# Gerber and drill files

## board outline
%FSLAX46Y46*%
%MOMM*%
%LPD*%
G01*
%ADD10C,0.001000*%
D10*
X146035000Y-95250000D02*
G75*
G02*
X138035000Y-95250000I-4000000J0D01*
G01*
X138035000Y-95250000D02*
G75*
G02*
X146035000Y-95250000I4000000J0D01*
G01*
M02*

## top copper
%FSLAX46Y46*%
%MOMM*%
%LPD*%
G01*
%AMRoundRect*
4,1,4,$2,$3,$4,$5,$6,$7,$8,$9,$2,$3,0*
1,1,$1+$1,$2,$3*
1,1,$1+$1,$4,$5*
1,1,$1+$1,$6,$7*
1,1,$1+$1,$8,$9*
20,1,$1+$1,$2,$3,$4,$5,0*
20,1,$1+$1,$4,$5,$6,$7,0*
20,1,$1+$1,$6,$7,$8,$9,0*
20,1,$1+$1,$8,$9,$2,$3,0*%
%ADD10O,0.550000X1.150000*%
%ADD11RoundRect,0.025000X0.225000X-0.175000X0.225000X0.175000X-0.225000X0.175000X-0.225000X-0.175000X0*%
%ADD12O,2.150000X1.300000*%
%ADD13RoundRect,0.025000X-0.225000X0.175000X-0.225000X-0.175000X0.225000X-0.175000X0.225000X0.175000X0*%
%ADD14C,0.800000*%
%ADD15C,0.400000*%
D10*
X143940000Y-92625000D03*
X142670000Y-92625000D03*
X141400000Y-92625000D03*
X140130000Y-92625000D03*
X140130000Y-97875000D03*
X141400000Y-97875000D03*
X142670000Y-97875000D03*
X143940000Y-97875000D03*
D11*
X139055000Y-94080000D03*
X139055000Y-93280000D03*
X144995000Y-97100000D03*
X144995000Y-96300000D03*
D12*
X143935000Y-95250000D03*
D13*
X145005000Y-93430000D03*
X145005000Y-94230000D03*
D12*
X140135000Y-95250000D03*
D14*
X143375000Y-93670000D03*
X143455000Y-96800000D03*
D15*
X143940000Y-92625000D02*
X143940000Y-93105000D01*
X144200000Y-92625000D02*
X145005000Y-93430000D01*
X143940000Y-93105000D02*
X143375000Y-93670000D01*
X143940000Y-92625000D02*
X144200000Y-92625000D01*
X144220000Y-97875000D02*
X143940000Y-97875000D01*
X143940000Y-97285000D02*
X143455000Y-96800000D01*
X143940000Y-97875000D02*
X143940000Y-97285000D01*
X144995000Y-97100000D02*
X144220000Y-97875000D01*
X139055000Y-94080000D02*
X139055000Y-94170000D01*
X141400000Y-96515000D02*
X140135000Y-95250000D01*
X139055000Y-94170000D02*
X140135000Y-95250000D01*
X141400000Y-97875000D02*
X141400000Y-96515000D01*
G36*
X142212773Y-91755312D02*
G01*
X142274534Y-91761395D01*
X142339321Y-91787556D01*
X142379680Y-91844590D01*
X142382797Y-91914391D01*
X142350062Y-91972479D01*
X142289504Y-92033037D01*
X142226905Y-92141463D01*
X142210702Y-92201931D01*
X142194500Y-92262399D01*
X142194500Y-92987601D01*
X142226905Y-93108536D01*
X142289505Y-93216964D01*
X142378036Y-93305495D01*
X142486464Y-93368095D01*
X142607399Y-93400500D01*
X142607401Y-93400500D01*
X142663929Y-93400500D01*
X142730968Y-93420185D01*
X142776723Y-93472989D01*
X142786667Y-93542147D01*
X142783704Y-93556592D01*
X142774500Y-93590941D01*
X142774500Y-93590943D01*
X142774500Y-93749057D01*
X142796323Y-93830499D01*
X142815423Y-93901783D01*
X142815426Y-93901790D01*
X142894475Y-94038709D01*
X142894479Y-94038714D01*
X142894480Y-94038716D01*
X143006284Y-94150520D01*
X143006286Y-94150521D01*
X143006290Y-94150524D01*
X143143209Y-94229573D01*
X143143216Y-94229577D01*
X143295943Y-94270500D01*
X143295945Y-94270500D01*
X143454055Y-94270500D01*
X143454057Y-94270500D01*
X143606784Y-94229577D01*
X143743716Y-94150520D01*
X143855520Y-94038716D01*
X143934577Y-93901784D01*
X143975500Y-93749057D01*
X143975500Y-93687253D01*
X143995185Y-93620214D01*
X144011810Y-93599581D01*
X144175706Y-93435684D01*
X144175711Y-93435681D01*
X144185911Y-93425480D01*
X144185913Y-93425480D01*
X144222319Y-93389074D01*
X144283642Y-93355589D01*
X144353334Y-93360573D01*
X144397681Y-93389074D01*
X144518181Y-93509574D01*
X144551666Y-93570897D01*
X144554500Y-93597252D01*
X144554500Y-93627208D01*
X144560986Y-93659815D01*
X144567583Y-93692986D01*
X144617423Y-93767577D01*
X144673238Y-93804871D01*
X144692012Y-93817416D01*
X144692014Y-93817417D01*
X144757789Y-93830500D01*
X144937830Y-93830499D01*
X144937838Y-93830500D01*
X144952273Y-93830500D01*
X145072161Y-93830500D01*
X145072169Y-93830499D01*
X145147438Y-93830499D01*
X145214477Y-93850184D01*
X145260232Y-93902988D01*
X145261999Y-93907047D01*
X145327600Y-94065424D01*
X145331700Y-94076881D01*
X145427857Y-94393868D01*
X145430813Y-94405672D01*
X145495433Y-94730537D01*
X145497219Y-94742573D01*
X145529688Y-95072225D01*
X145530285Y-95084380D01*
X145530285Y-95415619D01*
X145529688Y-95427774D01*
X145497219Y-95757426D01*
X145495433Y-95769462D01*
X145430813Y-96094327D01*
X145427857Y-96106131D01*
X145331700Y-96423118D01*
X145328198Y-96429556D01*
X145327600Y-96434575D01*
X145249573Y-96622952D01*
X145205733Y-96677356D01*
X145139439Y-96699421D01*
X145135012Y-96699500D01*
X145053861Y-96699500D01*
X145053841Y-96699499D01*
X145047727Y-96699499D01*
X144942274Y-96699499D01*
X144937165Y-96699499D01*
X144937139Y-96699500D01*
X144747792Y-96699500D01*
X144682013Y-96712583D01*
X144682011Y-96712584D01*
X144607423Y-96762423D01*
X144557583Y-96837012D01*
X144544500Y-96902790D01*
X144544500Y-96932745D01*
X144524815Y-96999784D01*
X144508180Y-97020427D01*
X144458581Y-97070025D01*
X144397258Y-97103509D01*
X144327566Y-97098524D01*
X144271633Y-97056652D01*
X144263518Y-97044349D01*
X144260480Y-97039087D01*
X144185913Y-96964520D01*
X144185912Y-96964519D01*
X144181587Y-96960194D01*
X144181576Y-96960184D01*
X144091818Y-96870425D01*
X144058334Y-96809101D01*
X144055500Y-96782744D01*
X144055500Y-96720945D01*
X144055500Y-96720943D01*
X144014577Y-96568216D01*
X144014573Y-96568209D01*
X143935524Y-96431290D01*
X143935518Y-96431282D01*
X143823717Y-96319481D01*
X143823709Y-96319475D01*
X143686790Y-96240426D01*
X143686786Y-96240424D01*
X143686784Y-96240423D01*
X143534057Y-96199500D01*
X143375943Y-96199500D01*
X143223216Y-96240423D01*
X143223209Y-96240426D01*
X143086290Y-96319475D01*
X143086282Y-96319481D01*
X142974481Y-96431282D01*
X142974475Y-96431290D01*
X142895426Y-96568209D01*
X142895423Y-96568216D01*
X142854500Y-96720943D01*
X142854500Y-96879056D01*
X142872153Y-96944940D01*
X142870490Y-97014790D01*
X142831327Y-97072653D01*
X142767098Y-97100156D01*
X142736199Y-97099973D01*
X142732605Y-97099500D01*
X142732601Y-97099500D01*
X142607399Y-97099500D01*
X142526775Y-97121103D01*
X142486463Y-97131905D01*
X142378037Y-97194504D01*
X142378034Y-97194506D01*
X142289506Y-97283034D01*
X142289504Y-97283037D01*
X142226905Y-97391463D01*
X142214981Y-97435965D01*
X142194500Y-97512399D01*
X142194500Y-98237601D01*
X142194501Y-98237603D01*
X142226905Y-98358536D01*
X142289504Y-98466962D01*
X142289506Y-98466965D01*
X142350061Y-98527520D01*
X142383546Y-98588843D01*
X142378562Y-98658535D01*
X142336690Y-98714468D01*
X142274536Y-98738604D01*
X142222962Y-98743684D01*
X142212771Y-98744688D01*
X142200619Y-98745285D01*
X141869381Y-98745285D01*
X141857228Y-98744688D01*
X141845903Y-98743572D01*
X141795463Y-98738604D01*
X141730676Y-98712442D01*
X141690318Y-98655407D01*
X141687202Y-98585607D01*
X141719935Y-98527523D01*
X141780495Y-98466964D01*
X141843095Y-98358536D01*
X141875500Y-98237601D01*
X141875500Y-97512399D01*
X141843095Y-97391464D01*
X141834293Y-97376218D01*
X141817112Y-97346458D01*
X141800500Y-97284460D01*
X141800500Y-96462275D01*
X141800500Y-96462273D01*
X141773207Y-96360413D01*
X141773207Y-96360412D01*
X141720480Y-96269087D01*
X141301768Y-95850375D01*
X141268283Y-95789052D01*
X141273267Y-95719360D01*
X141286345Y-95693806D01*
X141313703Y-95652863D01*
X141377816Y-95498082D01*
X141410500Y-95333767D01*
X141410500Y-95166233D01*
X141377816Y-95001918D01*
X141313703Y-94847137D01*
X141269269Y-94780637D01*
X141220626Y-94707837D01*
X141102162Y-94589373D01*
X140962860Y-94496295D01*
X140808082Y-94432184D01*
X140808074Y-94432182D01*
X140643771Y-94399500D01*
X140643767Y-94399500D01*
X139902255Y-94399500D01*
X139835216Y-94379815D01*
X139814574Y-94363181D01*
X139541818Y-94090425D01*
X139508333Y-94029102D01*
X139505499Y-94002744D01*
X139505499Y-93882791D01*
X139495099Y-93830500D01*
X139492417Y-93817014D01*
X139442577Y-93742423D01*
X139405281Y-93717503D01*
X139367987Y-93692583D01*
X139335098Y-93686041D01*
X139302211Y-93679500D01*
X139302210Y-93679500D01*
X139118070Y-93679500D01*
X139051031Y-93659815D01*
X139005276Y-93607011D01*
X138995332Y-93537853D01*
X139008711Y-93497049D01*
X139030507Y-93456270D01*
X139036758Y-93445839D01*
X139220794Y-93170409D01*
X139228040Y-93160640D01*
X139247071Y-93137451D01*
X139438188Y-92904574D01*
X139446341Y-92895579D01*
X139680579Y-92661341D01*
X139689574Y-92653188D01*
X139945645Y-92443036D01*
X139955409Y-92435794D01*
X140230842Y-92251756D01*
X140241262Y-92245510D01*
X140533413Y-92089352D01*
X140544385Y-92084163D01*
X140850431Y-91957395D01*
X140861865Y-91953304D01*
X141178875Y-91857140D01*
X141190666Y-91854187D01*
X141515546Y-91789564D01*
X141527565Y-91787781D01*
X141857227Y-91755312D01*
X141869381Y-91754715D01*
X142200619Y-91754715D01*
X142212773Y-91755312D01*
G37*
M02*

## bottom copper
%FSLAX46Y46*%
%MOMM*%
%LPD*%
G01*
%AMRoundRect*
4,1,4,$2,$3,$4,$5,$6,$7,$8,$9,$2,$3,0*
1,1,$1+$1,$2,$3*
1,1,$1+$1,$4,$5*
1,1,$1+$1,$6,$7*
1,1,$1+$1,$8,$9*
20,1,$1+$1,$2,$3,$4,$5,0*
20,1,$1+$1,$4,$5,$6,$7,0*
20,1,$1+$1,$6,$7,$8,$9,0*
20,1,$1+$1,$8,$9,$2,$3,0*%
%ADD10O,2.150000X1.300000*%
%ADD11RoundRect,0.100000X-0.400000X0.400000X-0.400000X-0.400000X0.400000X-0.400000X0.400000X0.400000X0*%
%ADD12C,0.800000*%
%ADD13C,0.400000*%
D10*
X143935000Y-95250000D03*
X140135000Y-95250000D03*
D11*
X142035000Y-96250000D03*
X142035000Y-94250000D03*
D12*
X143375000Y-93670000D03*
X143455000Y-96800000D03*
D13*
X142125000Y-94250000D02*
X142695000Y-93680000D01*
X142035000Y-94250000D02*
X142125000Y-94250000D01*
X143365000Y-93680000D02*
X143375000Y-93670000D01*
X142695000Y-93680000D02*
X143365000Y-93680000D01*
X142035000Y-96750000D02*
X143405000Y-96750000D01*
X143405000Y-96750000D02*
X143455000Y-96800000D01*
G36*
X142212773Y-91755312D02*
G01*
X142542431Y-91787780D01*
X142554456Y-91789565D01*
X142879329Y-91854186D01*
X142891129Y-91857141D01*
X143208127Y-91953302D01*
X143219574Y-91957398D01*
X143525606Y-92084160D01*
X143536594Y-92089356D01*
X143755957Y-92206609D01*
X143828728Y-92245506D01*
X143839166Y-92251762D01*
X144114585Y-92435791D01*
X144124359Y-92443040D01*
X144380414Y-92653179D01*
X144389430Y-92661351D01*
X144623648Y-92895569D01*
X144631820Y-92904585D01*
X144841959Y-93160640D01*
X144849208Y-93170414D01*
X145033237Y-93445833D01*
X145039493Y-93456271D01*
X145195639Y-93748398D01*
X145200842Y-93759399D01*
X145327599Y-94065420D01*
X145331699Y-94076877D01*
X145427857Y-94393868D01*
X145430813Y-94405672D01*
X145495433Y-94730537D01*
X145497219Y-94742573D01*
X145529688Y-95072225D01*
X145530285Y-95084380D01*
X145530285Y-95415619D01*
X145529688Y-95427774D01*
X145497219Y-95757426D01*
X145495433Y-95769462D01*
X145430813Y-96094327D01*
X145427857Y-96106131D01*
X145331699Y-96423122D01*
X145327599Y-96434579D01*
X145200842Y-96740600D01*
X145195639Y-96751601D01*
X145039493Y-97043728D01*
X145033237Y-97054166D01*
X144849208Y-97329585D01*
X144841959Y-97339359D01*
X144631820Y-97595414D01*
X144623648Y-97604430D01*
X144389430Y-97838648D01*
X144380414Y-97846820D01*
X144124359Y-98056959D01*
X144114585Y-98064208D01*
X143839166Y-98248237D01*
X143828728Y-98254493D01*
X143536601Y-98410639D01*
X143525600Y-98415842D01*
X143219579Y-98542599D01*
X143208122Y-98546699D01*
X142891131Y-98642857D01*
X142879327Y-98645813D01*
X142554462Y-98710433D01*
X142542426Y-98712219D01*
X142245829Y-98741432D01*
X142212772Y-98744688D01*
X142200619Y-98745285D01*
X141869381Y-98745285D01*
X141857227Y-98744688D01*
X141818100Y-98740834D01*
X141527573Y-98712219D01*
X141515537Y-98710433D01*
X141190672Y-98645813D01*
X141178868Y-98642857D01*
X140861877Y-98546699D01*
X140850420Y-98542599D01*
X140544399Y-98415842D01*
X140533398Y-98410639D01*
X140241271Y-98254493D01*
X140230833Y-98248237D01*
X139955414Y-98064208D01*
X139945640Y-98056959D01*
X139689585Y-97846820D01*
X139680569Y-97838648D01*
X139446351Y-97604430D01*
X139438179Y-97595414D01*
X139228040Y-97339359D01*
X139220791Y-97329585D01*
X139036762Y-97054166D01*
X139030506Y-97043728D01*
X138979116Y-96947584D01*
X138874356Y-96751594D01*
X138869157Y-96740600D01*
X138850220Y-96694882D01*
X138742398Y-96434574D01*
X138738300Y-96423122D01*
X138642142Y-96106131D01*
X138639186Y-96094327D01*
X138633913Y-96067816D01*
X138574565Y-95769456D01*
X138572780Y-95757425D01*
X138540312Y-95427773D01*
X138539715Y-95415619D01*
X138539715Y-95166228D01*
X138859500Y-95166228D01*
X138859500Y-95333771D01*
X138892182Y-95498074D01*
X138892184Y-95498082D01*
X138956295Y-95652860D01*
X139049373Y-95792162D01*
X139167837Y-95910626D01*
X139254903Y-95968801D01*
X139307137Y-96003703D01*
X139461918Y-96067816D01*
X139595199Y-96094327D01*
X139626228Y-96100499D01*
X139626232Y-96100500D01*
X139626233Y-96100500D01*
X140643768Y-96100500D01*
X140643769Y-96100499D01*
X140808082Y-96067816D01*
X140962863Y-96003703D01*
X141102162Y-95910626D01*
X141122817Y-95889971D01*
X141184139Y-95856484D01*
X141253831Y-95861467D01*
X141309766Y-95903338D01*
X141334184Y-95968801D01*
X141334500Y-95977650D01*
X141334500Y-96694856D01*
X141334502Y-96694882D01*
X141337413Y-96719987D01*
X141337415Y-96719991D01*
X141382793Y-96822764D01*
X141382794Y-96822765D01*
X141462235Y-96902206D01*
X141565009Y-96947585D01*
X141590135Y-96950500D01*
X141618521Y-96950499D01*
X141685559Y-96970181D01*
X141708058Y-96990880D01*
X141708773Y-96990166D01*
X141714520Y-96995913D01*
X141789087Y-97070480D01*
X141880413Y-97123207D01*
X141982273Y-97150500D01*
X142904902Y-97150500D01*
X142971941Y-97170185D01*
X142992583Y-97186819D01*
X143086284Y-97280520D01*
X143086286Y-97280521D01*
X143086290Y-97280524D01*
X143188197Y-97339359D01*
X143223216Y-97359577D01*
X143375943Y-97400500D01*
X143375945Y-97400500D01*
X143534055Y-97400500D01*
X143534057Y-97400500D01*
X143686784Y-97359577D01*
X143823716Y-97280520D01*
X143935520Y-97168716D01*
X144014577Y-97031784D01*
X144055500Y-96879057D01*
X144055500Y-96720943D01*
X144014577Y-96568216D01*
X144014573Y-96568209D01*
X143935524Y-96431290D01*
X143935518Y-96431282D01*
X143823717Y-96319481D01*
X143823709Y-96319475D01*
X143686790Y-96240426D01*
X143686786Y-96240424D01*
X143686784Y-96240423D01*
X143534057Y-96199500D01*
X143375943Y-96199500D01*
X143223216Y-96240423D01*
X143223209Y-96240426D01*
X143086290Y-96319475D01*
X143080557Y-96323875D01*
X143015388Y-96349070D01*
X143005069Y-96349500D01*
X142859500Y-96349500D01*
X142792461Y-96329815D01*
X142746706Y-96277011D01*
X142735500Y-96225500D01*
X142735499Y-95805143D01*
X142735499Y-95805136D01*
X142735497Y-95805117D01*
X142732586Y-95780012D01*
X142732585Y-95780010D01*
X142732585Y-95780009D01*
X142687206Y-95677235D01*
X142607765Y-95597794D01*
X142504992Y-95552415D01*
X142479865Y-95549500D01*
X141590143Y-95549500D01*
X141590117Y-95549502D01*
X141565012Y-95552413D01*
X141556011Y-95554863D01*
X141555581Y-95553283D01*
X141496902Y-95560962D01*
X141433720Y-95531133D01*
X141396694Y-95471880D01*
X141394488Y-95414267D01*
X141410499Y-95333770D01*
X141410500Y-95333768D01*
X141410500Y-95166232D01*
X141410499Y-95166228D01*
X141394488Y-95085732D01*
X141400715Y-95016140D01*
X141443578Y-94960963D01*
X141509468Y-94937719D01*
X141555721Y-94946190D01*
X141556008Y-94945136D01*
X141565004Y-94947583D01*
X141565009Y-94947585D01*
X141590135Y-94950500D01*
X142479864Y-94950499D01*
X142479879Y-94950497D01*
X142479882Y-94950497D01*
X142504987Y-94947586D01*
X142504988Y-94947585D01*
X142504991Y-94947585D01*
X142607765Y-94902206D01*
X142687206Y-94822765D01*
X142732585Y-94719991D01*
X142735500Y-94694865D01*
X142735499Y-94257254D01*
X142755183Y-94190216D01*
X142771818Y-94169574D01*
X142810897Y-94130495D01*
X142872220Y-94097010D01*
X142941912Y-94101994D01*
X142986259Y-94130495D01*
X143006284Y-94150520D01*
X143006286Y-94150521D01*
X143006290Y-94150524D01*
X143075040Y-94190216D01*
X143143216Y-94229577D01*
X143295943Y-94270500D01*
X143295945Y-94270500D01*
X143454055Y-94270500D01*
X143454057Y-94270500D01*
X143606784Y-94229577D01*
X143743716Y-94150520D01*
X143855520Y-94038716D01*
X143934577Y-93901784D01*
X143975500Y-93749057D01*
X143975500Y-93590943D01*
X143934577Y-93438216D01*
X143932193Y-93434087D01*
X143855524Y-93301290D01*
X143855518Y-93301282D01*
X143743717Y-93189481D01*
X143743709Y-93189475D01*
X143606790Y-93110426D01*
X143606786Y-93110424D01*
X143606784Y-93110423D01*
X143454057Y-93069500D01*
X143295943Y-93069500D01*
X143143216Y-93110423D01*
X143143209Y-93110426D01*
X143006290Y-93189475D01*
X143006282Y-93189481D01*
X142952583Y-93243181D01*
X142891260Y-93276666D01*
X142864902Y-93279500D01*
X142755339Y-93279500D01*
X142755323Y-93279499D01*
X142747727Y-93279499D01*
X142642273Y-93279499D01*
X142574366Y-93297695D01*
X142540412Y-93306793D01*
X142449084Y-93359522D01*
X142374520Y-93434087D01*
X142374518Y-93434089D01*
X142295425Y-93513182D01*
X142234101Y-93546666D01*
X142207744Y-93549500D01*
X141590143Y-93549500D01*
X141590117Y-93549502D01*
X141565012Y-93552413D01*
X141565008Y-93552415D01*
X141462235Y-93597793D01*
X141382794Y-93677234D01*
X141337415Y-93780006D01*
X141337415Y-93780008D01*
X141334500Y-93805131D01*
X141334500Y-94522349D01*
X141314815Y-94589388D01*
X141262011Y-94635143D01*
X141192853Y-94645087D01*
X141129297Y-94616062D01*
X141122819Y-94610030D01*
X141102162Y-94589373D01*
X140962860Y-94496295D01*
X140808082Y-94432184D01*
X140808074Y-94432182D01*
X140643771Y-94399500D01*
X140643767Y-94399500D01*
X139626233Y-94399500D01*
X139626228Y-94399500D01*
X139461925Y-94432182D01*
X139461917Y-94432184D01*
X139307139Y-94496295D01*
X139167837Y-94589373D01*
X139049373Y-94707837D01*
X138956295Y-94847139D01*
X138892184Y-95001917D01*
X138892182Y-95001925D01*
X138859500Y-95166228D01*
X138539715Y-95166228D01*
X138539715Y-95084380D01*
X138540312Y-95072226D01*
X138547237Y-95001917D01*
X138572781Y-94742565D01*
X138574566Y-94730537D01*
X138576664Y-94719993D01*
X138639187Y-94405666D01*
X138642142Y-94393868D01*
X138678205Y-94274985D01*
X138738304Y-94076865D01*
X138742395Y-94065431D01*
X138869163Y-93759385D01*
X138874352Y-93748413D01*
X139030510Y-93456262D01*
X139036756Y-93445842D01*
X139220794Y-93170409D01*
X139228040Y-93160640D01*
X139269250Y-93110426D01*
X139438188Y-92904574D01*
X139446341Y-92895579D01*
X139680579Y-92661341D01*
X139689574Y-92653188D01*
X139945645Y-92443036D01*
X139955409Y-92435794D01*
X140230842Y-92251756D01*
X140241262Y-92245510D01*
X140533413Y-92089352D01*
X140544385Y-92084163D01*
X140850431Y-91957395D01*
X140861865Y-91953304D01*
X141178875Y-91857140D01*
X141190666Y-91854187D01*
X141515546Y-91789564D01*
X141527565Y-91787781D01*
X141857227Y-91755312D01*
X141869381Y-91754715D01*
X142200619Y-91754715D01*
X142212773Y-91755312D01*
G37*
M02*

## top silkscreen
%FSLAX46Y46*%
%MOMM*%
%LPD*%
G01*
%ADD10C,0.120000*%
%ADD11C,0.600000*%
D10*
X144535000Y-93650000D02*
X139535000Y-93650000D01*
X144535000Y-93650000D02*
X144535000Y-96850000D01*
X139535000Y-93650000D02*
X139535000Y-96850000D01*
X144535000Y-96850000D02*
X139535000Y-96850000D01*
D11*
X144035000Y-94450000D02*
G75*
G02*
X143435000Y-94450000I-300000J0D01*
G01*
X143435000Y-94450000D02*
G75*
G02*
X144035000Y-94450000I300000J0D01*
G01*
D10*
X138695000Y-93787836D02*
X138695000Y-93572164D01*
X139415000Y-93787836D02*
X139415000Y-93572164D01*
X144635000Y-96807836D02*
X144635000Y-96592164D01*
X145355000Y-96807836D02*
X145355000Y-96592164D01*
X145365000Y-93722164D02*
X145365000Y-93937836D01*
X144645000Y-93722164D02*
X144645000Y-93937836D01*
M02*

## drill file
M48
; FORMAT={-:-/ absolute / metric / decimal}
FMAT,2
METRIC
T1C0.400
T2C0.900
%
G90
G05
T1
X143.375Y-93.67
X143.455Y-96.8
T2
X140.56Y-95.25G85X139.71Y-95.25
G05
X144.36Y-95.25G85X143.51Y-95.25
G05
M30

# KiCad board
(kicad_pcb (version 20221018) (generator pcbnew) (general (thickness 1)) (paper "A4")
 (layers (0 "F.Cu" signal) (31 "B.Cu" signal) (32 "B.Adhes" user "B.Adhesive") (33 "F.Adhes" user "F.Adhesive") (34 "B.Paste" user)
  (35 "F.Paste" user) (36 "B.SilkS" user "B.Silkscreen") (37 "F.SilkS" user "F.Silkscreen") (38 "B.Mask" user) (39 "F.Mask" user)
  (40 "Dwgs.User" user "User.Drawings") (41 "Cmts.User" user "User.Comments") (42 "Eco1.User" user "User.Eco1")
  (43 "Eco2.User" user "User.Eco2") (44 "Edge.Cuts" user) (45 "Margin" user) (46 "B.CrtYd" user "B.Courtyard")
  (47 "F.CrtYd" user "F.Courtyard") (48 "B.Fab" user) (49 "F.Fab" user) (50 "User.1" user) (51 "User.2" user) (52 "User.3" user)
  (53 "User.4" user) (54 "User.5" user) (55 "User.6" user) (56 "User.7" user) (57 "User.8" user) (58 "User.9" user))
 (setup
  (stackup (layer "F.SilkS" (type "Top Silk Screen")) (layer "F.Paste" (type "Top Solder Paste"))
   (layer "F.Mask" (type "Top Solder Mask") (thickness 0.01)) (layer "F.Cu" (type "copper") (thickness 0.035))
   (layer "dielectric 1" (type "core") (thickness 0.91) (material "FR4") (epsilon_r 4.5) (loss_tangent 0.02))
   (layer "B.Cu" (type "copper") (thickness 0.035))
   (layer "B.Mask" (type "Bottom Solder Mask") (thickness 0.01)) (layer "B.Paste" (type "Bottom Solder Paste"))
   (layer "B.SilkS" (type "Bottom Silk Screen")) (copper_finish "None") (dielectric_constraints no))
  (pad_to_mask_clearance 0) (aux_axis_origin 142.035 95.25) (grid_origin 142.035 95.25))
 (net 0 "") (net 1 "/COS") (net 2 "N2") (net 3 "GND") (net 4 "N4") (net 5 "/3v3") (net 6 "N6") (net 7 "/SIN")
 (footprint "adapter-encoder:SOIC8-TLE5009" (layer "F.Cu") (at 142.035 95.25 -90)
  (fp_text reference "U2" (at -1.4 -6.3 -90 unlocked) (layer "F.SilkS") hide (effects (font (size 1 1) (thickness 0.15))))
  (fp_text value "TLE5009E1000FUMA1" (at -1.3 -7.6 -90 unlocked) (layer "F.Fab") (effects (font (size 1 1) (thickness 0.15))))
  (fp_line (start -1.6 -2.5) (end -1.6 2.5) (stroke (width 0.12) (type default)) (layer "F.SilkS"))
  (fp_line (start -1.6 -2.5) (end 1.6 -2.5) (stroke (width 0.12) (type default)) (layer "F.SilkS"))
  (fp_line (start -1.6 2.5) (end 1.6 2.5) (stroke (width 0.12) (type default)) (layer "F.SilkS"))
  (fp_line (start 1.6 -2.5) (end 1.6 2.5) (stroke (width 0.12) (type default)) (layer "F.SilkS"))
  (fp_circle (center -0.8 -1.7) (end -0.5 -1.7) (stroke (width 0.6) (type default)) (fill none) (layer "F.SilkS"))
  (pad "1" smd oval (at -2.625 -1.905) (size 0.55 1.15) (layers "F.Cu" "F.Paste" "F.Mask") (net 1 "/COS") (solder_mask_margin 0.0508))
  (pad "2" smd oval (at -2.625 -0.635) (size 0.55 1.15) (layers "F.Cu" "F.Paste" "F.Mask") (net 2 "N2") (solder_mask_margin 0.0508))
  (pad "3" smd oval (at -2.625 0.635) (size 0.55 1.15) (layers "F.Cu" "F.Paste" "F.Mask") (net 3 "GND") (solder_mask_margin 0.0508))
  (pad "4" smd oval (at -2.625 1.905) (size 0.55 1.15) (layers "F.Cu" "F.Paste" "F.Mask") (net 3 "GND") (solder_mask_margin 0.0508))
  (pad "5" smd oval (at 2.625 1.905) (size 0.55 1.15) (layers "F.Cu" "F.Paste" "F.Mask") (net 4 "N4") (solder_mask_margin 0.0508))
  (pad "6" smd oval (at 2.625 0.635) (size 0.55 1.15) (layers "F.Cu" "F.Paste" "F.Mask") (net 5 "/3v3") (solder_mask_margin 0.0508))
  (pad "7" smd oval (at 2.625 -0.635) (size 0.55 1.15) (layers "F.Cu" "F.Paste" "F.Mask") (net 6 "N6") (solder_mask_margin 0.0508))
  (pad "8" smd oval (at 2.625 -1.905) (size 0.55 1.15) (layers "F.Cu" "F.Paste" "F.Mask") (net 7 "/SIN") (solder_mask_margin 0.0508)))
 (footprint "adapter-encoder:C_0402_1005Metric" (layer "F.Cu") (at 139.055 93.68 90)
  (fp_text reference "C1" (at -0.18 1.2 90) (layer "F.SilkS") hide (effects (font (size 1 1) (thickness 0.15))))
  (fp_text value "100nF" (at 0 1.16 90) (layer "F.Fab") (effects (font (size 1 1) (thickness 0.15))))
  (fp_line (start -0.107836 -0.36) (end 0.107836 -0.36) (stroke (width 0.12) (type solid)) (layer "F.SilkS"))
  (fp_line (start -0.107836 0.36) (end 0.107836 0.36) (stroke (width 0.12) (type solid)) (layer "F.SilkS"))
  (pad "1" smd roundrect (at -0.4 0 90) (size 0.4 0.5) (layers "F.Cu" "F.Paste" "F.Mask") (roundrect_rratio 0.0625) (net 5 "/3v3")
   (solder_mask_margin 0.0508))
  (pad "2" smd roundrect (at 0.4 0 90) (size 0.4 0.5) (layers "F.Cu" "F.Paste" "F.Mask") (roundrect_rratio 0.0625) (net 3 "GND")
   (solder_mask_margin 0.0508)))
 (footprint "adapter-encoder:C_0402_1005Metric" (layer "F.Cu") (at 144.995 96.7 90)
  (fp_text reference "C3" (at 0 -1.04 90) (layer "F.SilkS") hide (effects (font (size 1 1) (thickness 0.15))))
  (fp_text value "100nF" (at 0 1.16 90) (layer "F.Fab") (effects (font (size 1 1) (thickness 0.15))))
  (fp_line (start -0.107836 -0.36) (end 0.107836 -0.36) (stroke (width 0.12) (type solid)) (layer "F.SilkS"))
  (fp_line (start -0.107836 0.36) (end 0.107836 0.36) (stroke (width 0.12) (type solid)) (layer "F.SilkS"))
  (pad "1" smd roundrect (at -0.4 0 90) (size 0.4 0.5) (layers "F.Cu" "F.Paste" "F.Mask") (roundrect_rratio 0.0625) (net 7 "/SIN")
   (solder_mask_margin 0.0508))
  (pad "2" smd roundrect (at 0.4 0 90) (size 0.4 0.5) (layers "F.Cu" "F.Paste" "F.Mask") (roundrect_rratio 0.0625) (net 3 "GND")
   (solder_mask_margin 0.0508)))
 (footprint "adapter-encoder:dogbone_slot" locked (layer "F.Cu") (at 143.935 95.25 180)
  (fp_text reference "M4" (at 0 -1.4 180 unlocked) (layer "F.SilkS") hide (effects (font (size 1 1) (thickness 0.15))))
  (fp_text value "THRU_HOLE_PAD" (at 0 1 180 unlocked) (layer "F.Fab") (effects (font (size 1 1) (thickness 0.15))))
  (pad "1" thru_hole oval locked (at 0 0 180) (size 2.15 1.3) (drill oval 1.75 0.9) (layers "*.Cu" "*.Mask") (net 3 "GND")
   (thermal_bridge_angle 45)))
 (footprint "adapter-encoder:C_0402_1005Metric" (layer "F.Cu") (at 145.005 93.83 -90)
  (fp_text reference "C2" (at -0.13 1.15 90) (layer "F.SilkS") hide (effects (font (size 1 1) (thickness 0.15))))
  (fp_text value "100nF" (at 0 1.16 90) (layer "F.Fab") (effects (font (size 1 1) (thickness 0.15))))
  (fp_line (start -0.107836 -0.36) (end 0.107836 -0.36) (stroke (width 0.12) (type solid)) (layer "F.SilkS"))
  (fp_line (start -0.107836 0.36) (end 0.107836 0.36) (stroke (width 0.12) (type solid)) (layer "F.SilkS"))
  (pad "1" smd roundrect (at -0.4 0 270) (size 0.4 0.5) (layers "F.Cu" "F.Paste" "F.Mask") (roundrect_rratio 0.0625) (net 1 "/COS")
   (solder_mask_margin 0.0508))
  (pad "2" smd roundrect (at 0.4 0 270) (size 0.4 0.5) (layers "F.Cu" "F.Paste" "F.Mask") (roundrect_rratio 0.0625) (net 3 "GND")
   (solder_mask_margin 0.0508)))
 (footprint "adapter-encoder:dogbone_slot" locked (layer "F.Cu") (at 140.135 95.25 180)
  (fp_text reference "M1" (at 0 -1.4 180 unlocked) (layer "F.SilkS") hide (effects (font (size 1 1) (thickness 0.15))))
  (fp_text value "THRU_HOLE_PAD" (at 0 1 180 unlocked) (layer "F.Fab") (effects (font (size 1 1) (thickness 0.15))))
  (pad "1" thru_hole oval locked (at 0 0 180) (size 2.15 1.3) (drill oval 1.75 0.9) (layers "*.Cu" "*.Mask") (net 5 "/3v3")
   (thermal_bridge_angle 45)))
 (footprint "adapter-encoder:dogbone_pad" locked (layer "B.Cu") (at 142.035 96.25 -90)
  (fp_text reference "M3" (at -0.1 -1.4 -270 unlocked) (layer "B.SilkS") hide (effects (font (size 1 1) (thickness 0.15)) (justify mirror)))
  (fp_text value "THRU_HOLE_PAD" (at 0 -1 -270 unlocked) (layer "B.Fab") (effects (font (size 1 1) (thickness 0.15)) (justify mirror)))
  (pad "1" smd roundrect locked (at 0 0 270) (size 1 1) (layers "B.Cu" "B.Paste" "B.Mask") (roundrect_rratio 0.1) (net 7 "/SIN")
   (thermal_bridge_angle 45)))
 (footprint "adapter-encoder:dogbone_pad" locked (layer "B.Cu") (at 142.035 94.25 -90)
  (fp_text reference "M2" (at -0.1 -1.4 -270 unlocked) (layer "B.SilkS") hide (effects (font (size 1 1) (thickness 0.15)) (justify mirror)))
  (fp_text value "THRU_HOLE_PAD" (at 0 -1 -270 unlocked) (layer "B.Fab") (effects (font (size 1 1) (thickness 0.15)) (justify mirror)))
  (pad "1" smd roundrect locked (at 0 0 270) (size 1 1) (layers "B.Cu" "B.Paste" "B.Mask") (roundrect_rratio 0.1) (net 1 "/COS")
   (thermal_bridge_angle 45)))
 (gr_circle locked (center 142.035 95.25) (end 146.035 95.25) (stroke (width 0.001) (type solid)) (fill none) (layer "Edge.Cuts"))
 (segment (start 143.94 92.625) (end 143.94 93.105) (width 0.4) (layer "F.Cu") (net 1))
 (segment (start 144.2 92.625) (end 145.005 93.43) (width 0.4) (layer "F.Cu") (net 1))
 (segment (start 143.94 93.105) (end 143.375 93.67) (width 0.4) (layer "F.Cu") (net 1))
 (segment (start 143.94 92.625) (end 144.2 92.625) (width 0.4) (layer "F.Cu") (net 1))
 (via (at 143.375 93.67) (size 0.8) (drill 0.4) (layers "F.Cu" "B.Cu") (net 1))
 (segment (start 142.125 94.25) (end 142.695 93.68) (width 0.4) (layer "B.Cu") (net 1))
 (segment (start 142.035 94.25) (end 142.125 94.25) (width 0.4) (layer "B.Cu") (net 1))
 (segment (start 143.365 93.68) (end 143.375 93.67) (width 0.4) (layer "B.Cu") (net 1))
 (segment (start 142.695 93.68) (end 143.365 93.68) (width 0.4) (layer "B.Cu") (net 1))
 (segment (start 144.22 97.875) (end 143.94 97.875) (width 0.4) (layer "F.Cu") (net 7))
 (segment (start 143.94 97.285) (end 143.455 96.8) (width 0.4) (layer "F.Cu") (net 7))
 (segment (start 143.94 97.875) (end 143.94 97.285) (width 0.4) (layer "F.Cu") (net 7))
 (segment (start 144.995 97.1) (end 144.22 97.875) (width 0.4) (layer "F.Cu") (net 7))
 (via (at 143.455 96.8) (size 0.8) (drill 0.4) (layers "F.Cu" "B.Cu") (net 7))
 (segment (start 142.035 96.75) (end 143.405 96.75) (width 0.4) (layer "B.Cu") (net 7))
 (segment (start 143.405 96.75) (end 143.455 96.8) (width 0.4) (layer "B.Cu") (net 7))
 (segment (start 139.055 94.08) (end 139.055 94.17) (width 0.4) (layer "F.Cu") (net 5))
 (segment (start 141.4 96.515) (end 140.135 95.25) (width 0.4) (layer "F.Cu") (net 5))
 (segment (start 139.055 94.17) (end 140.135 95.25) (width 0.4) (layer "F.Cu") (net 5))
 (segment (start 141.4 97.875) (end 141.4 96.515) (width 0.4) (layer "F.Cu") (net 5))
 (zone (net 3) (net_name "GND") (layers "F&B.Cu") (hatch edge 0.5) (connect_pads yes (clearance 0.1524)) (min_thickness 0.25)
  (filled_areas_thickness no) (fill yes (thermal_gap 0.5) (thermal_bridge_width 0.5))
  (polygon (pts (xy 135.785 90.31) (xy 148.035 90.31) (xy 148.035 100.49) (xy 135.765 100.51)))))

